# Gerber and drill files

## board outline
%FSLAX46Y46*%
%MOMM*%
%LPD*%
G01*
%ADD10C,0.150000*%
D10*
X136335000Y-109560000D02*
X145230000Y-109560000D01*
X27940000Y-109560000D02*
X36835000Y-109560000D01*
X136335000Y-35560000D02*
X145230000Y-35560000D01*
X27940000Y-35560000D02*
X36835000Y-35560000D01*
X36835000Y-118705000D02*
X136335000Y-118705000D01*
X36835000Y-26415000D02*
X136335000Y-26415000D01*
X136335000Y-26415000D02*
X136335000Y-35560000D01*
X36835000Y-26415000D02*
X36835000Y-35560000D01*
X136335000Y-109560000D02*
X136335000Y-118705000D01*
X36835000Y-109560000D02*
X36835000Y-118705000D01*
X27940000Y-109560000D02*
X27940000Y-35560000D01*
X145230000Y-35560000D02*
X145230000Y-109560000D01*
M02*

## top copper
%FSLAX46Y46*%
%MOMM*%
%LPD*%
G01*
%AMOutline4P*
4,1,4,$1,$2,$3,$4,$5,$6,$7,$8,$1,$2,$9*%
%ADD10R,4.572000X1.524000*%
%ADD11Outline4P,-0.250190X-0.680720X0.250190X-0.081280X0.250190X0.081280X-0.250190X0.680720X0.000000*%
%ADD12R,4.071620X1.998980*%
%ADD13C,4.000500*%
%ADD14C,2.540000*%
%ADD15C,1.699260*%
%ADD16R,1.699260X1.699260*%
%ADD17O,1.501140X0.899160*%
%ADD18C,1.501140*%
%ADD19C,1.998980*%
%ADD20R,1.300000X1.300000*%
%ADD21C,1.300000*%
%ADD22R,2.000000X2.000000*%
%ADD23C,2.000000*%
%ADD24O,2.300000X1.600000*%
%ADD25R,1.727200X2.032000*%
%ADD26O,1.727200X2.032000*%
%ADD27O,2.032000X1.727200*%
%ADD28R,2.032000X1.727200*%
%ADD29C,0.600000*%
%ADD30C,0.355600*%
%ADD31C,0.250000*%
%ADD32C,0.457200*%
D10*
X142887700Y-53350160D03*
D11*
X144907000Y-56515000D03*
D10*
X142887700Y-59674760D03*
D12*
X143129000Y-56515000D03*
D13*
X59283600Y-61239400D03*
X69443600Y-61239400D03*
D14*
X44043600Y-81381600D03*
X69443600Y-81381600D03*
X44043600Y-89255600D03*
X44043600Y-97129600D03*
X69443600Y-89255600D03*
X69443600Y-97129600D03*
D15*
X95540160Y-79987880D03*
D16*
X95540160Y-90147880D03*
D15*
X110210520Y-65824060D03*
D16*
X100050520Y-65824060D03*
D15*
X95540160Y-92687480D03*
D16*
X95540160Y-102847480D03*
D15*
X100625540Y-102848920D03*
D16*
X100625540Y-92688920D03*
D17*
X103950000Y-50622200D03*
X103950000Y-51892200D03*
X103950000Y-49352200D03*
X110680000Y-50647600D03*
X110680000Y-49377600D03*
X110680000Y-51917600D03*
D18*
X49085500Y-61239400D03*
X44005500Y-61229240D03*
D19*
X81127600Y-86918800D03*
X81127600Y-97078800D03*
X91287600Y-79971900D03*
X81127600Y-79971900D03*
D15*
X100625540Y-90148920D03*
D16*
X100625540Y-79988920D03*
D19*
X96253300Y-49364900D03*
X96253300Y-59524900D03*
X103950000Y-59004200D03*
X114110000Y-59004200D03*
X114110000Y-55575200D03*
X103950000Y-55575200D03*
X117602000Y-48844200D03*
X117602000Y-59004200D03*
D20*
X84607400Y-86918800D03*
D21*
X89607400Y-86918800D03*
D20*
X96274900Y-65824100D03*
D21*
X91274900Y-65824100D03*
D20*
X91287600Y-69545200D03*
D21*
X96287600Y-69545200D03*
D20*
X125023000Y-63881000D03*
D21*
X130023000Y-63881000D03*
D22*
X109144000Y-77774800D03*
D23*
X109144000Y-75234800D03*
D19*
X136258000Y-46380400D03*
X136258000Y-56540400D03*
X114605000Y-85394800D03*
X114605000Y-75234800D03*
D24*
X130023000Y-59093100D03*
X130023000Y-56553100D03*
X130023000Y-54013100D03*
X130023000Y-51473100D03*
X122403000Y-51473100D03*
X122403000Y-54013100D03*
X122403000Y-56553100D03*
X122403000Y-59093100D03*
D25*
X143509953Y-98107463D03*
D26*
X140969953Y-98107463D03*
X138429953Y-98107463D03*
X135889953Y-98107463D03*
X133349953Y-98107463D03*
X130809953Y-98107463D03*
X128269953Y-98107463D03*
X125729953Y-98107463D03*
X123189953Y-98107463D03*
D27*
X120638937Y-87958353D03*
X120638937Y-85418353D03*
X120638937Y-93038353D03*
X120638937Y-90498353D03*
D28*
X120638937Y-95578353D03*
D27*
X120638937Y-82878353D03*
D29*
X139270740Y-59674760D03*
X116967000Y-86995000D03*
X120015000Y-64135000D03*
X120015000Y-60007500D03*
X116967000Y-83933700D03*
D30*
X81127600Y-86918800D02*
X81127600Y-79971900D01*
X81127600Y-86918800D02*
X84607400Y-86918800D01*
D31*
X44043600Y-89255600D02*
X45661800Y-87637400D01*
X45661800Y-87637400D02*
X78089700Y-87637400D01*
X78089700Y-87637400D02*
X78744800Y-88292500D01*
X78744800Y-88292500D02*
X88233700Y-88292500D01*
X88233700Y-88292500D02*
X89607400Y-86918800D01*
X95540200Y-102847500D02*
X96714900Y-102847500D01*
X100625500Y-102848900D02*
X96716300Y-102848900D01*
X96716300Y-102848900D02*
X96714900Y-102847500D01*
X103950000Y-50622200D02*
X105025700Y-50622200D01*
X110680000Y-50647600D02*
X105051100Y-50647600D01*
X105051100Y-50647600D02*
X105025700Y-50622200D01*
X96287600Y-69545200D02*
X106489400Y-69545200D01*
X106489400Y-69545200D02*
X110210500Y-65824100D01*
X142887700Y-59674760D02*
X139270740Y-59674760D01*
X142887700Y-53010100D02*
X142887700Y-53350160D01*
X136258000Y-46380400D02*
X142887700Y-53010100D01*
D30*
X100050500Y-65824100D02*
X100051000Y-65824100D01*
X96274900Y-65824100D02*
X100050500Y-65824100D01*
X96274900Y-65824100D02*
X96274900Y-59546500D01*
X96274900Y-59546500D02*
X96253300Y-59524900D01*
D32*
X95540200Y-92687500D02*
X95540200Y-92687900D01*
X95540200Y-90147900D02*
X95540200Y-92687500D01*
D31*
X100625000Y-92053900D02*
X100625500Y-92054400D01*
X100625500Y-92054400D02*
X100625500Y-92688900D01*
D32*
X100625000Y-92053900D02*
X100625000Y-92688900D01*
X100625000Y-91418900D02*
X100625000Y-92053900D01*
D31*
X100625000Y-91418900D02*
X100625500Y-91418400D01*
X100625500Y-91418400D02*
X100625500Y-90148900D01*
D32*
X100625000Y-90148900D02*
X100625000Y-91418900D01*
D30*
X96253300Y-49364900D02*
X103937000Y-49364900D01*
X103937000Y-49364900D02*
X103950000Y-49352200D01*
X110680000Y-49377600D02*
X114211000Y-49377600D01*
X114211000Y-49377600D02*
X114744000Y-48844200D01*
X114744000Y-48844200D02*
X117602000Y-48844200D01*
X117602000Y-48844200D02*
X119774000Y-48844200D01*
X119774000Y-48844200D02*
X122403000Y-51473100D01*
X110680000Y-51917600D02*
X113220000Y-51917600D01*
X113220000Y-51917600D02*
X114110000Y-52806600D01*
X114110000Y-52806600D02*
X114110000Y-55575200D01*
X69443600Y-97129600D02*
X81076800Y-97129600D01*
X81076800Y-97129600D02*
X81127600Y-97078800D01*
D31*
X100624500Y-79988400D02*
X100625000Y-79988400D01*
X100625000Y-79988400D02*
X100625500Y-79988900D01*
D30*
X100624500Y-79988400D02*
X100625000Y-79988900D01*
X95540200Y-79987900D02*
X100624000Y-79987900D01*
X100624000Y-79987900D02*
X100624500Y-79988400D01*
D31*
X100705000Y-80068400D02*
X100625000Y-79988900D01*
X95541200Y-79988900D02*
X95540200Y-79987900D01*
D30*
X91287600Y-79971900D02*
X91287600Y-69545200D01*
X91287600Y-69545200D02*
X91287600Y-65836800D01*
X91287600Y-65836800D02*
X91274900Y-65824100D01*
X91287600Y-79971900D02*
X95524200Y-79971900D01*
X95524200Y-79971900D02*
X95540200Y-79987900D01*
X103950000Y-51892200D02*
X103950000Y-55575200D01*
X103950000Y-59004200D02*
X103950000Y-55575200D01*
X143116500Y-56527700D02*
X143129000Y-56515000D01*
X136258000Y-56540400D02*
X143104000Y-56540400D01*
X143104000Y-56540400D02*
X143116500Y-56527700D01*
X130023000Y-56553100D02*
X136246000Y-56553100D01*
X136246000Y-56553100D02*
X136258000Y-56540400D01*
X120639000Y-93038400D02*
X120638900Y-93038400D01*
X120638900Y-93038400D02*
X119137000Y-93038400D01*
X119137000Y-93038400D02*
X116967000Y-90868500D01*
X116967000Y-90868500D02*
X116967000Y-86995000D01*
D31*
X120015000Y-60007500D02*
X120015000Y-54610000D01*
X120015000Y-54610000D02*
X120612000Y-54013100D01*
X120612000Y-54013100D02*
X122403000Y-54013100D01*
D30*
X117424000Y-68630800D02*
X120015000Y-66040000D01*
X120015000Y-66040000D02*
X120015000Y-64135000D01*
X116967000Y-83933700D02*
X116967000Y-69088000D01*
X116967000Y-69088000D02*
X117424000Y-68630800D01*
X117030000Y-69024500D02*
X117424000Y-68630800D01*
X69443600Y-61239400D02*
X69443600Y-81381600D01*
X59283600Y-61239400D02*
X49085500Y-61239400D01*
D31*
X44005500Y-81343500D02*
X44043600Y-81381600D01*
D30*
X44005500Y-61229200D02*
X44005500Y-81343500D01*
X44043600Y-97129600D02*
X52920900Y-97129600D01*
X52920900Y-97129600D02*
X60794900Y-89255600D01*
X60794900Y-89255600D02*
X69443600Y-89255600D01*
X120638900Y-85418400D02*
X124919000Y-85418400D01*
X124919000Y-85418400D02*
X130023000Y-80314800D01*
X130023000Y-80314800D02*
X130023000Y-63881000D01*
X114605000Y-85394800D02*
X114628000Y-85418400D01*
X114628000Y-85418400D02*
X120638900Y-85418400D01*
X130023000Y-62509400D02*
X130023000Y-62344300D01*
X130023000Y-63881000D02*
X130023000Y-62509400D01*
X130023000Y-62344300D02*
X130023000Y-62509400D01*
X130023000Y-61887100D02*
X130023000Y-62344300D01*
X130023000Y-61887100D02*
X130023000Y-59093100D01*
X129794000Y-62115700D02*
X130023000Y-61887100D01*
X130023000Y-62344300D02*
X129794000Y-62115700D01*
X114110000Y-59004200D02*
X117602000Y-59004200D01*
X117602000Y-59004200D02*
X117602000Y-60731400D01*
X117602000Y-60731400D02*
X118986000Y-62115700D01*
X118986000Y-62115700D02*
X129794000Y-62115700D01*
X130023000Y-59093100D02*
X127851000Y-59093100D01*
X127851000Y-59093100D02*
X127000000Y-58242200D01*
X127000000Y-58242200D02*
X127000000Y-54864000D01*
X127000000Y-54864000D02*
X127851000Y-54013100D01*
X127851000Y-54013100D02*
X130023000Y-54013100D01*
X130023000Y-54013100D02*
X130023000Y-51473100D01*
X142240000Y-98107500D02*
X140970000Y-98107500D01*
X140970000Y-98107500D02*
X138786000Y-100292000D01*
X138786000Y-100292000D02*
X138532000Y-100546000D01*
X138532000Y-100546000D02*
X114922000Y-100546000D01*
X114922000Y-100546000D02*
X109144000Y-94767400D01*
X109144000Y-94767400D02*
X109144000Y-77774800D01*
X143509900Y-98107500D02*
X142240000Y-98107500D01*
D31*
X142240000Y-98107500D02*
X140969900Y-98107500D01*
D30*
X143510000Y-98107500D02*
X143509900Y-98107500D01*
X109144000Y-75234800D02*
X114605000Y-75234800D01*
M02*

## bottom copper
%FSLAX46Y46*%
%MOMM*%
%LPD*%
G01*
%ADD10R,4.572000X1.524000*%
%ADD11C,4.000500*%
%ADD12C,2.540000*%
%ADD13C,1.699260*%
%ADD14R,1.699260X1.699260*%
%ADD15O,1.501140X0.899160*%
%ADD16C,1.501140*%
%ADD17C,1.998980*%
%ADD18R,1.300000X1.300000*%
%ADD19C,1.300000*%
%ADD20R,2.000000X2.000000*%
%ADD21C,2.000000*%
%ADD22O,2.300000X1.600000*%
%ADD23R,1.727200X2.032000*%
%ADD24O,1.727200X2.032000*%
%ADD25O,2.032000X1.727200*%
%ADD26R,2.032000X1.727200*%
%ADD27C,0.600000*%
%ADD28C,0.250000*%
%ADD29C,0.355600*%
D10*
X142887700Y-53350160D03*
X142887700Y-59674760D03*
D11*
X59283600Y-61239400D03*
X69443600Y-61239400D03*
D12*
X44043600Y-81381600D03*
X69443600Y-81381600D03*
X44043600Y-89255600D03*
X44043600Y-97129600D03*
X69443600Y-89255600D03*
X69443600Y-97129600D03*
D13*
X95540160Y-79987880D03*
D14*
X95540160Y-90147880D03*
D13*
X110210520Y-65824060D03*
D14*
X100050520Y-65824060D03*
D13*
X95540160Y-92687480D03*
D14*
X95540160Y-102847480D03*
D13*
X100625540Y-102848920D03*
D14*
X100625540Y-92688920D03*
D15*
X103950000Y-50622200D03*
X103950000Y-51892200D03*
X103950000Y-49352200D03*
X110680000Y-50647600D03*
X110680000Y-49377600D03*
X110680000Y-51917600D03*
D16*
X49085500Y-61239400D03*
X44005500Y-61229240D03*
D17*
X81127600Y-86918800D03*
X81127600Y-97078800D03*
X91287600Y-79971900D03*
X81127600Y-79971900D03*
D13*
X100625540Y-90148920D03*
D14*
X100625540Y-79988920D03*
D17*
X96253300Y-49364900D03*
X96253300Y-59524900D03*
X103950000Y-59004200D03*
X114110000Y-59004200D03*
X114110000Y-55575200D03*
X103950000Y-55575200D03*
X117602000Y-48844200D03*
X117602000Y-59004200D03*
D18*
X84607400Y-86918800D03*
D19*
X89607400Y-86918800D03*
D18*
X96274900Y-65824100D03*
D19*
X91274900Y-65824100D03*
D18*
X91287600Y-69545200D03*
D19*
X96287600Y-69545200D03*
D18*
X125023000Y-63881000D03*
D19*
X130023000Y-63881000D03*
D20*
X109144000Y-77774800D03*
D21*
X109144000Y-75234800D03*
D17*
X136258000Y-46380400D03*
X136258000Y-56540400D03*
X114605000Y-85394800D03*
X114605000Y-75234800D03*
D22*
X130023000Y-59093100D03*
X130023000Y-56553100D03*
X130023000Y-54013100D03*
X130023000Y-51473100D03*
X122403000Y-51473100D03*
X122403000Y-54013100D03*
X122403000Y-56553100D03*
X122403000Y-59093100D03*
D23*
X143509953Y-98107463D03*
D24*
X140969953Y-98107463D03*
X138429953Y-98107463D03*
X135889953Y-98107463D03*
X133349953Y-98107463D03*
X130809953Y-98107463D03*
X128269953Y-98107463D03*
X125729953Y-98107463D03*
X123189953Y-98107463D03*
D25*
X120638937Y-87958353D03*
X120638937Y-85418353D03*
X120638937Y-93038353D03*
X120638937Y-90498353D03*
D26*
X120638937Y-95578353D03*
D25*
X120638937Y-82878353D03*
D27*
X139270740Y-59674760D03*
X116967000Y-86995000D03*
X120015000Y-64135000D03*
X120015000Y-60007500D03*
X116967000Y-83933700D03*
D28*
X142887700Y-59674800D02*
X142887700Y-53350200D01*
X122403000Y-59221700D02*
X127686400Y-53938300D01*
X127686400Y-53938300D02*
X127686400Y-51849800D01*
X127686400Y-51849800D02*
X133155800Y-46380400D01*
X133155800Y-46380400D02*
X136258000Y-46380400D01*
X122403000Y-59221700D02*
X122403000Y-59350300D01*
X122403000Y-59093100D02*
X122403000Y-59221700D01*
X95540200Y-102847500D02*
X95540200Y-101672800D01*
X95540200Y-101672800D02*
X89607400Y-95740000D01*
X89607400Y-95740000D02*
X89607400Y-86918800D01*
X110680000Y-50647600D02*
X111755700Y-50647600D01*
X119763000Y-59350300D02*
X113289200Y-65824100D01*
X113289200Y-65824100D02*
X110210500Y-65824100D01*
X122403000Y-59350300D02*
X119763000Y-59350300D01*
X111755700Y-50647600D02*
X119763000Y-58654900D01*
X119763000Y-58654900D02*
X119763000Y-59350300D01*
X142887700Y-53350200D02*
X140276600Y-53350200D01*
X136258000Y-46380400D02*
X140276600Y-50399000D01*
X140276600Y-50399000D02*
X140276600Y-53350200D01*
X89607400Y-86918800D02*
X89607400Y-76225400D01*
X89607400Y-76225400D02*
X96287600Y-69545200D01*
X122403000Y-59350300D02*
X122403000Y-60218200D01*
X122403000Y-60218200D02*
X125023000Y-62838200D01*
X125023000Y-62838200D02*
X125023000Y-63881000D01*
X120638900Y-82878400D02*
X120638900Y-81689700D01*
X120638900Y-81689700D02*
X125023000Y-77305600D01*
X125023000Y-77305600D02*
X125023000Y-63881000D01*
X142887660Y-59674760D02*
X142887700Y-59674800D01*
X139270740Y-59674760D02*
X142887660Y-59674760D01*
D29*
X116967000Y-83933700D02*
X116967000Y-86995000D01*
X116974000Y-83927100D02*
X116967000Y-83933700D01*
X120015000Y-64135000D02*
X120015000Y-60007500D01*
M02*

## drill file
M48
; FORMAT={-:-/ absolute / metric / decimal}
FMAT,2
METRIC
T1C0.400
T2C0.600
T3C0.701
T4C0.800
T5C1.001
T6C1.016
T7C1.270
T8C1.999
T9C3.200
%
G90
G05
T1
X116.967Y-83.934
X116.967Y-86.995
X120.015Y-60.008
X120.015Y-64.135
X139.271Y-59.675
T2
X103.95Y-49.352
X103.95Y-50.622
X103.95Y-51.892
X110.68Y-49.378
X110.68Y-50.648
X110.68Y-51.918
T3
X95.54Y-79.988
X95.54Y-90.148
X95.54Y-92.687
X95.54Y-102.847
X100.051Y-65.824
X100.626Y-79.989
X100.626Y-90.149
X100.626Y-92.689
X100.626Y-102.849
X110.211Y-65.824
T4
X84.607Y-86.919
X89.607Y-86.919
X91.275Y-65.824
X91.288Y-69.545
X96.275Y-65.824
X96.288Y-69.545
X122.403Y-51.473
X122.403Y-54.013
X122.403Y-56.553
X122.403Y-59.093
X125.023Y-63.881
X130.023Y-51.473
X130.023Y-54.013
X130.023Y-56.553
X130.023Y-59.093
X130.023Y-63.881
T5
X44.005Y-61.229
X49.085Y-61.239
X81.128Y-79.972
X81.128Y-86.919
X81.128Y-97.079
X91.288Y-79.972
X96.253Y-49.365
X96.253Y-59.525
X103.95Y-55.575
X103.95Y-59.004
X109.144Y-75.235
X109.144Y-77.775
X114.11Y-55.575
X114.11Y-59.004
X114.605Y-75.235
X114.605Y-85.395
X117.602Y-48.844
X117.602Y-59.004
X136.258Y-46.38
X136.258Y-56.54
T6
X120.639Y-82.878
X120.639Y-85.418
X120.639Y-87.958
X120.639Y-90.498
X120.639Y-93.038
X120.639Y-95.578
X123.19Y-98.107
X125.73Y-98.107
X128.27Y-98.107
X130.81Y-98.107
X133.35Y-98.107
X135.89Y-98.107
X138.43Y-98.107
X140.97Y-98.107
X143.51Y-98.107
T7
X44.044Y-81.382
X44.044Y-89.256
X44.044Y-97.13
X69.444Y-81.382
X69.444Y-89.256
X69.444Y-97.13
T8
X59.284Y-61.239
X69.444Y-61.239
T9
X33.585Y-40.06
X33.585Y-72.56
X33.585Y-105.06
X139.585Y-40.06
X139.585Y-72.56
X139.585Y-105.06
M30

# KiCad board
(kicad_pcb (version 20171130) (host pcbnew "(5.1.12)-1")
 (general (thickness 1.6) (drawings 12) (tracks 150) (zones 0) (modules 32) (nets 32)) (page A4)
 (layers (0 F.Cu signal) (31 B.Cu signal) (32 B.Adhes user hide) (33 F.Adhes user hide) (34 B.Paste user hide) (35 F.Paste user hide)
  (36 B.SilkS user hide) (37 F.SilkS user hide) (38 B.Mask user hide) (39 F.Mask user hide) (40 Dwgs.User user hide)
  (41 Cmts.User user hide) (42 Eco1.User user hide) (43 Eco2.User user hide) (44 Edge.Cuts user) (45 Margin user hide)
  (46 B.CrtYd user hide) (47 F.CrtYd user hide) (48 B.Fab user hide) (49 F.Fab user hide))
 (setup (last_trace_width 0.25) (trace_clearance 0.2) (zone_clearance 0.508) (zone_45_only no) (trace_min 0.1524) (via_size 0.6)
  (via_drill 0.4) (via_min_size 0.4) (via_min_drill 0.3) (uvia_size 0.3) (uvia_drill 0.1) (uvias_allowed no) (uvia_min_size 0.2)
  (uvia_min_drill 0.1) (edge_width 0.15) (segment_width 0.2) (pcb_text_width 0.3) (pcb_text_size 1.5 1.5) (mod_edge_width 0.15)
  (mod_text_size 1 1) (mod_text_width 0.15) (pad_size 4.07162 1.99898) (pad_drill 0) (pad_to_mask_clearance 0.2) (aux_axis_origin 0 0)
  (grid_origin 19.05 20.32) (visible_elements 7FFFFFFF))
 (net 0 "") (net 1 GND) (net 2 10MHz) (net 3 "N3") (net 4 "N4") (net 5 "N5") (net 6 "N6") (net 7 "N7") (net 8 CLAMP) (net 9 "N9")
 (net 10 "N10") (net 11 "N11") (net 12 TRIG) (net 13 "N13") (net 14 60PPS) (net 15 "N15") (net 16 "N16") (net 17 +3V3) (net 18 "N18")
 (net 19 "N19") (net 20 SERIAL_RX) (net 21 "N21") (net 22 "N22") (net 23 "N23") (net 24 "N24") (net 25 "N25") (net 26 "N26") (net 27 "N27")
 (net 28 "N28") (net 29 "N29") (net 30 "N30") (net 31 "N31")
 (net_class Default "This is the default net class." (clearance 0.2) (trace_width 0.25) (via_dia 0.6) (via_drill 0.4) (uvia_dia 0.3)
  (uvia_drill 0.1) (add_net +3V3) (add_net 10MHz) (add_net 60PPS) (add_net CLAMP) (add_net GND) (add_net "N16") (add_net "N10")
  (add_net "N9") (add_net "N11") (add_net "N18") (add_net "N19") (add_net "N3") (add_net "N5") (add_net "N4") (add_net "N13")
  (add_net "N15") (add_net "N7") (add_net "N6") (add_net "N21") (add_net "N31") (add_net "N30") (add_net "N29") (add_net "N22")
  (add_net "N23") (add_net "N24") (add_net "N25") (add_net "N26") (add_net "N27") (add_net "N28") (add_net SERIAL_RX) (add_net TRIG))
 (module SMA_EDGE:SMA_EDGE (layer F.Cu) (at 151.765 55.245)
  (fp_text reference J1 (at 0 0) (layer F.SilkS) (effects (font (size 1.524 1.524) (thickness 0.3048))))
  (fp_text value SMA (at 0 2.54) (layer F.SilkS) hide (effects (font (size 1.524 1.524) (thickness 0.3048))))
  (pad 0 connect rect (at -8.8773 -1.89484) (size 4.572 1.524) (layers *.Cu F.Mask) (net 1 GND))
  (pad 1 connect trapezoid (at -6.858 1.27) (size 0.50038 0.762) (rect_delta 0.59944 0) (layers F.Cu F.Mask) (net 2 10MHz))
  (pad 2 connect rect (at -8.8773 4.42976) (size 4.572 1.524) (layers *.Cu F.Mask) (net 1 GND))
  (pad 1 connect rect (at -8.636 1.27) (size 4.07162 1.99898) (layers F.Cu F.Mask) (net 2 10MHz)))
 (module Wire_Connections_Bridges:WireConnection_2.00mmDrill (layer F.Cu) (at 59.2836 61.2394)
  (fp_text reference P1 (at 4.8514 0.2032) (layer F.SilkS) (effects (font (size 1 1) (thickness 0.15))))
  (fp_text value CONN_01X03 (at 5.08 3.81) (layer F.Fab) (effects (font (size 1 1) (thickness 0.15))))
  (pad 1 thru_hole circle (at 0 0) (size 4.0005 4.0005) (drill 1.99898) (layers *.Cu *.Mask F.SilkS) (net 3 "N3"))
  (pad 2 thru_hole circle (at 10.16 0) (size 4.0005 4.0005) (drill 1.99898) (layers *.Cu *.Mask F.SilkS) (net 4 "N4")))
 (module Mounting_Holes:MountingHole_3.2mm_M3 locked (layer F.Cu) (at 139.585 105.06)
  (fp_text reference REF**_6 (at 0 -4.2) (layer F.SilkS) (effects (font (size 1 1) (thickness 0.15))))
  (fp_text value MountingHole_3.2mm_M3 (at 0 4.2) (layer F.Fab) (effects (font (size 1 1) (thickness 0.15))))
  (pad 1 np_thru_hole circle (at 0 0) (size 3.2 3.2) (drill 3.2) (layers *.Cu *.Mask F.SilkS)))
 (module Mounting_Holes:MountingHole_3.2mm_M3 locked (layer F.Cu) (at 139.585 72.56)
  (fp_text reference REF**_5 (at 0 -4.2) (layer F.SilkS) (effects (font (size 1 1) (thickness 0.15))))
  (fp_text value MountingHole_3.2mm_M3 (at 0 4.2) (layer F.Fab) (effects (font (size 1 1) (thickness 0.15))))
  (pad 1 np_thru_hole circle (at 0 0) (size 3.2 3.2) (drill 3.2) (layers *.Cu *.Mask F.SilkS)))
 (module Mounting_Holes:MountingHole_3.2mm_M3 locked (layer F.Cu) (at 33.585 105.06)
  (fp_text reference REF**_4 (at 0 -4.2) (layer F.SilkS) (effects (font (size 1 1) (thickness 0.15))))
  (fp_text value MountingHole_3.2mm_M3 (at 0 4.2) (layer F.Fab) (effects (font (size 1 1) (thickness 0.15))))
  (pad 1 np_thru_hole circle (at 0 0) (size 3.2 3.2) (drill 3.2) (layers *.Cu *.Mask F.SilkS)))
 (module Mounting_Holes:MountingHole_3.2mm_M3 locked (layer F.Cu) (at 33.585 72.56)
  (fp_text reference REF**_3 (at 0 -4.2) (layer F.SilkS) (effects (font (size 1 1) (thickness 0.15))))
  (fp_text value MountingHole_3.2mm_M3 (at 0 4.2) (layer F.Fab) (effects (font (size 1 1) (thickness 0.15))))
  (pad 1 np_thru_hole circle (at 0 0) (size 3.2 3.2) (drill 3.2) (layers *.Cu *.Mask F.SilkS)))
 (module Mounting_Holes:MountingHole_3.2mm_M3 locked (layer F.Cu) (at 139.585 40.06)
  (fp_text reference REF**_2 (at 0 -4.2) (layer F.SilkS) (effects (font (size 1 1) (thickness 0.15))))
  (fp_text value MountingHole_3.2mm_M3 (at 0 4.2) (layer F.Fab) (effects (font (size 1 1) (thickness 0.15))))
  (pad 1 np_thru_hole circle (at 0 0) (size 3.2 3.2) (drill 3.2) (layers *.Cu *.Mask F.SilkS)))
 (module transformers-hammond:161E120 (layer F.Cu) (at 41.5036 71.2216)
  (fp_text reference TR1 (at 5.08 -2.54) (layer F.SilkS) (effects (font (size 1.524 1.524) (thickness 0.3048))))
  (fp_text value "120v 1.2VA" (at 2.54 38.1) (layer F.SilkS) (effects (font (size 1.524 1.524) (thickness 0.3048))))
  (pad 1 thru_hole circle (at 2.54 10.16) (size 2.54 2.54) (drill 1.27) (layers *.Cu *.Mask F.SilkS) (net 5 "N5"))
  (pad 2 thru_hole circle (at 27.94 10.16) (size 2.54 2.54) (drill 1.27) (layers *.Cu *.SilkS *.Mask) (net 4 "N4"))
  (pad 3 thru_hole circle (at 2.54 18.034) (size 2.54 2.54) (drill 1.27) (layers *.Cu *.SilkS *.Mask) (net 1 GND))
  (pad 4 thru_hole circle (at 2.54 25.908) (size 2.54 2.54) (drill 1.27) (layers *.Cu *.SilkS *.Mask) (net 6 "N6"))
  (pad 5 thru_hole circle (at 27.94 18.034) (size 2.54 2.54) (drill 1.27) (layers *.Cu *.SilkS *.Mask) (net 6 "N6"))
  (pad 6 thru_hole circle (at 27.94 25.908) (size 2.54 2.54) (drill 1.27) (layers *.Cu *.SilkS *.Mask) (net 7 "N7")))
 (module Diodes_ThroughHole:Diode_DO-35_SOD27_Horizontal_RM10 (layer F.Cu) (at 95.5427 90.1484 90)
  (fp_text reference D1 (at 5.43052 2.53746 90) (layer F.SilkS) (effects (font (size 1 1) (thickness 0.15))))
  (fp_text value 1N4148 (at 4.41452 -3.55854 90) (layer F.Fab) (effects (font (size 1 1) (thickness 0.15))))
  (pad 2 thru_hole circle (at 10.16052 -0.00254 270) (size 1.69926 1.69926) (drill 0.70104) (layers *.Cu *.Mask F.SilkS) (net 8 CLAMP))
  (pad 1 thru_hole rect (at 0.00052 -0.00254 270) (size 1.69926 1.69926) (drill 0.70104) (layers *.Cu *.Mask F.SilkS) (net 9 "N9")))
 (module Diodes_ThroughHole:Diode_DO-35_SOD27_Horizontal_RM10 (layer F.Cu) (at 100.05 65.8266)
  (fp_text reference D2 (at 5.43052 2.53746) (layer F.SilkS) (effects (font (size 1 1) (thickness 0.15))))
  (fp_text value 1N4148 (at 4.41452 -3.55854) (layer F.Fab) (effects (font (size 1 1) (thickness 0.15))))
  (pad 2 thru_hole circle (at 10.16052 -0.00254 180) (size 1.69926 1.69926) (drill 0.70104) (layers *.Cu *.Mask F.SilkS) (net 1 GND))
  (pad 1 thru_hole rect (at 0.00052 -0.00254 180) (size 1.69926 1.69926) (drill 0.70104) (layers *.Cu *.Mask F.SilkS) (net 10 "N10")))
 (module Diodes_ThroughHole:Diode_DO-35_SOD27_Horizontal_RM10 (layer F.Cu) (at 95.5427 102.848 90)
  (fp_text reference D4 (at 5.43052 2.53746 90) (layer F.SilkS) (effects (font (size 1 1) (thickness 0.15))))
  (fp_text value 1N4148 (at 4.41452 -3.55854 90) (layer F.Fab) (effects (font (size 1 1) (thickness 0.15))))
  (pad 2 thru_hole circle (at 10.16052 -0.00254 270) (size 1.69926 1.69926) (drill 0.70104) (layers *.Cu *.Mask F.SilkS) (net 9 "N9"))
  (pad 1 thru_hole rect (at 0.00052 -0.00254 270) (size 1.69926 1.69926) (drill 0.70104) (layers *.Cu *.Mask F.SilkS) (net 1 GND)))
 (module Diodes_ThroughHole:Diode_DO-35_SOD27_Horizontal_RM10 (layer F.Cu) (at 100.623 92.6884 270)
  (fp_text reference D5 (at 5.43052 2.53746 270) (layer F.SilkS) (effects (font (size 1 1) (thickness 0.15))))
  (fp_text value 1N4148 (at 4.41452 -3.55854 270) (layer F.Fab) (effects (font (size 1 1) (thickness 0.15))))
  (pad 2 thru_hole circle (at 10.16052 -0.00254 90) (size 1.69926 1.69926) (drill 0.70104) (layers *.Cu *.Mask F.SilkS) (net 1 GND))
  (pad 1 thru_hole rect (at 0.00052 -0.00254 90) (size 1.69926 1.69926) (drill 0.70104) (layers *.Cu *.Mask F.SilkS) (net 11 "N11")))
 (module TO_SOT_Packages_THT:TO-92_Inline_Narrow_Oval (layer F.Cu) (at 103.95 49.3522 270)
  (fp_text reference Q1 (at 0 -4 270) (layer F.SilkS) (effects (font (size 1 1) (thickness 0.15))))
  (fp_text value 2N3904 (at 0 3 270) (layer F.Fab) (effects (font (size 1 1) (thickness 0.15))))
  (pad 2 thru_hole oval (at 1.27 0 90) (size 0.89916 1.50114) (drill 0.6) (layers *.Cu *.Mask F.SilkS) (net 1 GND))
  (pad 3 thru_hole oval (at 2.54 0 90) (size 0.89916 1.50114) (drill 0.6) (layers *.Cu *.Mask F.SilkS) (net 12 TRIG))
  (pad 1 thru_hole oval (at 0 0 90) (size 0.89916 1.50114) (drill 0.6) (layers *.Cu *.Mask F.SilkS) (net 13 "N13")))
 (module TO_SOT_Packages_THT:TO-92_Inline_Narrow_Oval (layer F.Cu) (at 110.68 51.9176 90)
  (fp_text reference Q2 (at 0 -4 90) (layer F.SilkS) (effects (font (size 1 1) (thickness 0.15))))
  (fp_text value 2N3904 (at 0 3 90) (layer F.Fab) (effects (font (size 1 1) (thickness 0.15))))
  (pad 2 thru_hole oval (at 1.27 0 270) (size 0.89916 1.50114) (drill 0.6) (layers *.Cu *.Mask F.SilkS) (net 1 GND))
  (pad 3 thru_hole oval (at 2.54 0 270) (size 0.89916 1.50114) (drill 0.6) (layers *.Cu *.Mask F.SilkS) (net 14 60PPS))
  (pad 1 thru_hole oval (at 0 0 270) (size 0.89916 1.50114) (drill 0.6) (layers *.Cu *.Mask F.SilkS) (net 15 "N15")))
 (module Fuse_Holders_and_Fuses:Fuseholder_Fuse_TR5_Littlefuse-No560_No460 (layer F.Cu) (at 46.5455 61.2394 180)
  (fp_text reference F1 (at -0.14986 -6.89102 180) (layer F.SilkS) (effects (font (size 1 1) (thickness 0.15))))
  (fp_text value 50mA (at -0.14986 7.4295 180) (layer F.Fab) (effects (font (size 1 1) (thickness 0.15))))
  (pad 1 thru_hole circle (at -2.54 0 180) (size 1.50114 1.50114) (drill 1.00076) (layers *.Cu *.Mask F.SilkS) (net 3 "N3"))
  (pad 2 thru_hole circle (at 2.54 0.01016 180) (size 1.50114 1.50114) (drill 1.00076) (layers *.Cu *.Mask F.SilkS) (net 5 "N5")))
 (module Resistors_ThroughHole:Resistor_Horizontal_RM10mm (layer F.Cu) (at 81.1276 86.9188 270)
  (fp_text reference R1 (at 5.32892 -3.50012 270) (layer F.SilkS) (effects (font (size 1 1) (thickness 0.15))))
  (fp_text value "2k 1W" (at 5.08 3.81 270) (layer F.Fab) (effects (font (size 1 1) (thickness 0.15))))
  (pad 1 thru_hole circle (at 0 0 270) (size 1.99898 1.99898) (drill 1.00076) (layers *.Cu *.SilkS *.Mask) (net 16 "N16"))
  (pad 2 thru_hole circle (at 10.16 0 270) (size 1.99898 1.99898) (drill 1.00076) (layers *.Cu *.SilkS *.Mask) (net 7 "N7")))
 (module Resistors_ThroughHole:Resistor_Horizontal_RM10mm (layer F.Cu) (at 91.2876 79.9719 180)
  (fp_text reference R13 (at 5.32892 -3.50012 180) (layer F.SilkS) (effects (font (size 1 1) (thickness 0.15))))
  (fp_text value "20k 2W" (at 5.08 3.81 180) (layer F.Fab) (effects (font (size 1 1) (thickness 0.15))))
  (pad 1 thru_hole circle (at 0 0 180) (size 1.99898 1.99898) (drill 1.00076) (layers *.Cu *.SilkS *.Mask) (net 8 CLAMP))
  (pad 2 thru_hole circle (at 10.16 0 180) (size 1.99898 1.99898) (drill 1.00076) (layers *.Cu *.SilkS *.Mask) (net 16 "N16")))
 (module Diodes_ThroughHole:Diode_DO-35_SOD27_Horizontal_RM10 (layer F.Cu) (at 100.623 79.9884 270)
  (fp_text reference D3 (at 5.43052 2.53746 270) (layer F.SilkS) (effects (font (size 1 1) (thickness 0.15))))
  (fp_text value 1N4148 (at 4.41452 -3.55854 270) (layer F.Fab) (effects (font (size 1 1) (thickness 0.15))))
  (pad 2 thru_hole circle (at 10.16052 -0.00254 90) (size 1.69926 1.69926) (drill 0.70104) (layers *.Cu *.Mask F.SilkS) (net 11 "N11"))
  (pad 1 thru_hole rect (at 0.00052 -0.00254 90) (size 1.69926 1.69926) (drill 0.70104) (layers *.Cu *.Mask F.SilkS) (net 8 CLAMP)))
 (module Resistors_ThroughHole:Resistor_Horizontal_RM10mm (layer F.Cu) (at 96.2533 49.3649 270)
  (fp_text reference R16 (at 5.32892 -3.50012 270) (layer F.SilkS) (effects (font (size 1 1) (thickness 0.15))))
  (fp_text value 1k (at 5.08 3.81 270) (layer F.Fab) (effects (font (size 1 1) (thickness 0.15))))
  (pad 1 thru_hole circle (at 0 0 270) (size 1.99898 1.99898) (drill 1.00076) (layers *.Cu *.SilkS *.Mask) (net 13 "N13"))
  (pad 2 thru_hole circle (at 10.16 0 270) (size 1.99898 1.99898) (drill 1.00076) (layers *.Cu *.SilkS *.Mask) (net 10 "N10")))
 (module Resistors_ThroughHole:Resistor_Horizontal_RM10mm (layer F.Cu) (at 103.95 59.0042)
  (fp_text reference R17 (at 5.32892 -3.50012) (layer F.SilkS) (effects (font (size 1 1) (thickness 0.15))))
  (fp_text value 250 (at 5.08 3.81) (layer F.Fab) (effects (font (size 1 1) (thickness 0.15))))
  (pad 1 thru_hole circle (at 0 0) (size 1.99898 1.99898) (drill 1.00076) (layers *.Cu *.SilkS *.Mask) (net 12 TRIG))
  (pad 2 thru_hole circle (at 10.16 0) (size 1.99898 1.99898) (drill 1.00076) (layers *.Cu *.SilkS *.Mask) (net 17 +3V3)))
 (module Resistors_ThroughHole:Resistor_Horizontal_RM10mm (layer F.Cu) (at 114.11 55.5752 180)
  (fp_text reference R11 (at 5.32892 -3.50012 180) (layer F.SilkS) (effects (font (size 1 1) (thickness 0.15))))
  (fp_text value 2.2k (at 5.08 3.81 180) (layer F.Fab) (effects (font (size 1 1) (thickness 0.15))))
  (pad 1 thru_hole circle (at 0 0 180) (size 1.99898 1.99898) (drill 1.00076) (layers *.Cu *.SilkS *.Mask) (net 15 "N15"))
  (pad 2 thru_hole circle (at 10.16 0 180) (size 1.99898 1.99898) (drill 1.00076) (layers *.Cu *.SilkS *.Mask) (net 12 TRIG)))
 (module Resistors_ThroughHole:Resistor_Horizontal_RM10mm (layer F.Cu) (at 117.602 48.8442 270)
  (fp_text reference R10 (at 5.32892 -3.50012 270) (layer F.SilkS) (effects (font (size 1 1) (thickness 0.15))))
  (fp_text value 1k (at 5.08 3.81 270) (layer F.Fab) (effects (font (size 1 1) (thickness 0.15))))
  (pad 1 thru_hole circle (at 0 0 270) (size 1.99898 1.99898) (drill 1.00076) (layers *.Cu *.SilkS *.Mask) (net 14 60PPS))
  (pad 2 thru_hole circle (at 10.16 0 270) (size 1.99898 1.99898) (drill 1.00076) (layers *.Cu *.SilkS *.Mask) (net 17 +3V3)))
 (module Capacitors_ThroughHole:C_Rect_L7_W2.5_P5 (layer F.Cu) (at 84.6074 86.9188)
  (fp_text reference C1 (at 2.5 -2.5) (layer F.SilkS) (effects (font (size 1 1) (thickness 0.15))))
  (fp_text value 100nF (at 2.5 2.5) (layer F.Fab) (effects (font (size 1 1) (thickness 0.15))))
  (pad 1 thru_hole rect (at 0 0) (size 1.3 1.3) (drill 0.8) (layers *.Cu *.Mask F.SilkS) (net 16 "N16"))
  (pad 2 thru_hole circle (at 5 0) (size 1.3 1.3) (drill 0.8) (layers *.Cu *.Mask F.SilkS) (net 1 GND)))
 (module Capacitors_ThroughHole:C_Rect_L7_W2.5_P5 (layer F.Cu) (at 96.2749 65.8241 180)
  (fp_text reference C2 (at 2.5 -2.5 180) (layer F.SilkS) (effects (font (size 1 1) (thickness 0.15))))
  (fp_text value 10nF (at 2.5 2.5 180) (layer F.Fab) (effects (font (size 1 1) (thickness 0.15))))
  (pad 1 thru_hole rect (at 0 0 180) (size 1.3 1.3) (drill 0.8) (layers *.Cu *.Mask F.SilkS) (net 10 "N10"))
  (pad 2 thru_hole circle (at 5 0 180) (size 1.3 1.3) (drill 0.8) (layers *.Cu *.Mask F.SilkS) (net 8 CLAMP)))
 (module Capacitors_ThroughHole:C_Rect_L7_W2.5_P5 (layer F.Cu) (at 91.2876 69.5452)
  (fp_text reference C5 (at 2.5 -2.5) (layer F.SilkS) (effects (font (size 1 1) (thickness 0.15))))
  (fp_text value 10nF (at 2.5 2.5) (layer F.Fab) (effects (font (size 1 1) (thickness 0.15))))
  (pad 1 thru_hole rect (at 0 0) (size 1.3 1.3) (drill 0.8) (layers *.Cu *.Mask F.SilkS) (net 8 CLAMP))
  (pad 2 thru_hole circle (at 5 0) (size 1.3 1.3) (drill 0.8) (layers *.Cu *.Mask F.SilkS) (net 1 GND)))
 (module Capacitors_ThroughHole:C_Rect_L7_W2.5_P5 (layer F.Cu) (at 125.023 63.881)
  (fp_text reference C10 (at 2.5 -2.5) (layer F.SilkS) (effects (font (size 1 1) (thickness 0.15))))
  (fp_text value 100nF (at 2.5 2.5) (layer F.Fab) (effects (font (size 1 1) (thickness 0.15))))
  (pad 1 thru_hole rect (at 0 0) (size 1.3 1.3) (drill 0.8) (layers *.Cu *.Mask F.SilkS) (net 1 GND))
  (pad 2 thru_hole circle (at 5 0) (size 1.3 1.3) (drill 0.8) (layers *.Cu *.Mask F.SilkS) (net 17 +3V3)))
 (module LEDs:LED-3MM (layer F.Cu) (at 109.144 77.7748 90)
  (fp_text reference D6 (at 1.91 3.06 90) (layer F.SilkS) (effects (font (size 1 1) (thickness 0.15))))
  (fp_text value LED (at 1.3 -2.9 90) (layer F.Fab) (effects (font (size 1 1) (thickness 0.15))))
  (pad 1 thru_hole rect (at 0 0 180) (size 2 2) (drill 1.00076) (layers *.Cu *.Mask F.SilkS) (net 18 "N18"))
  (pad 2 thru_hole circle (at 2.54 0 90) (size 2 2) (drill 1.00076) (layers *.Cu *.Mask F.SilkS) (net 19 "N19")))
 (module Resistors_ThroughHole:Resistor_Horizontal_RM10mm (layer F.Cu) (at 136.258 46.3804 270)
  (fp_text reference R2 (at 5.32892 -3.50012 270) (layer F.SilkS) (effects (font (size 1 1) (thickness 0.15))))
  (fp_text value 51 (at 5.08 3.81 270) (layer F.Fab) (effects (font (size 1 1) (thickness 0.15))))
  (pad 1 thru_hole circle (at 0 0 270) (size 1.99898 1.99898) (drill 1.00076) (layers *.Cu *.SilkS *.Mask) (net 1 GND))
  (pad 2 thru_hole circle (at 10.16 0 270) (size 1.99898 1.99898) (drill 1.00076) (layers *.Cu *.SilkS *.Mask) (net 2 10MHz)))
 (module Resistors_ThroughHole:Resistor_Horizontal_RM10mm (layer F.Cu) (at 114.605 85.3948 90)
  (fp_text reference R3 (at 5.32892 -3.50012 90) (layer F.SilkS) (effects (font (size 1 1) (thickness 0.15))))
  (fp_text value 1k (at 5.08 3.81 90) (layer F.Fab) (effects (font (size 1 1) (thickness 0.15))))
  (pad 1 thru_hole circle (at 0 0 90) (size 1.99898 1.99898) (drill 1.00076) (layers *.Cu *.SilkS *.Mask) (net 17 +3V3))
  (pad 2 thru_hole circle (at 10.16 0 90) (size 1.99898 1.99898) (drill 1.00076) (layers *.Cu *.SilkS *.Mask) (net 19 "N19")))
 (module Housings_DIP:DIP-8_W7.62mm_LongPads (layer F.Cu) (at 130.023 59.0931 180)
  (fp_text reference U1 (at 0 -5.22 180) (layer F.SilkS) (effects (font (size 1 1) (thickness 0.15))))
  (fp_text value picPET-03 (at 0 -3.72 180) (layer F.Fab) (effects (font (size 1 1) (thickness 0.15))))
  (pad 1 thru_hole oval (at 0 0 180) (size 2.3 1.6) (drill 0.8) (layers *.Cu *.Mask F.SilkS) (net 17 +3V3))
  (pad 2 thru_hole oval (at 0 2.54 180) (size 2.3 1.6) (drill 0.8) (layers *.Cu *.Mask F.SilkS) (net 2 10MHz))
  (pad 3 thru_hole oval (at 0 5.08 180) (size 2.3 1.6) (drill 0.8) (layers *.Cu *.Mask F.SilkS) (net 17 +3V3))
  (pad 4 thru_hole oval (at 0 7.62 180) (size 2.3 1.6) (drill 0.8) (layers *.Cu *.Mask F.SilkS) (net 17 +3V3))
  (pad 5 thru_hole oval (at 7.62 7.62 180) (size 2.3 1.6) (drill 0.8) (layers *.Cu *.Mask F.SilkS) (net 14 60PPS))
  (pad 6 thru_hole oval (at 7.62 5.08 180) (size 2.3 1.6) (drill 0.8) (layers *.Cu *.Mask F.SilkS) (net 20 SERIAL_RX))
  (pad 7 thru_hole oval (at 7.62 2.54 180) (size 2.3 1.6) (drill 0.8) (layers *.Cu *.Mask F.SilkS) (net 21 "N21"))
  (pad 8 thru_hole oval (at 7.62 0 180) (size 2.3 1.6) (drill 0.8) (layers *.Cu *.Mask F.SilkS) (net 1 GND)))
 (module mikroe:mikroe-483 (layer F.Cu) (at 145.277 99.8854 180)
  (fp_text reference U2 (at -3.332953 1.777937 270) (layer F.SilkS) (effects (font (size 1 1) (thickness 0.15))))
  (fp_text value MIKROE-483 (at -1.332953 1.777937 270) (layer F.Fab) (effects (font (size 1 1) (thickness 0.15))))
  (pad 3-1 thru_hole rect (at 1.767047 1.777937 270) (size 2.032 1.7272) (drill 1.016) (layers *.Cu *.Mask F.SilkS) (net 18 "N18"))
  (pad 3-2 thru_hole oval (at 4.307047 1.777937 270) (size 2.032 1.7272) (drill 1.016) (layers *.Cu *.Mask F.SilkS) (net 18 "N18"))
  (pad 3-3 thru_hole oval (at 6.847047 1.777937 270) (size 2.032 1.7272) (drill 1.016) (layers *.Cu *.Mask F.SilkS) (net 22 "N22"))
  (pad 3-4 thru_hole oval (at 9.387047 1.777937 270) (size 2.032 1.7272) (drill 1.016) (layers *.Cu *.Mask F.SilkS) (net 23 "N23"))
  (pad 3-5 thru_hole oval (at 11.927047 1.777937 90) (size 2.032 1.7272) (drill 1.016) (layers *.Cu *.Mask F.SilkS) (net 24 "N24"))
  (pad 3-6 thru_hole oval (at 14.467047 1.777937 270) (size 2.032 1.7272) (drill 1.016) (layers *.Cu *.Mask F.SilkS) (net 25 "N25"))
  (pad 3-7 thru_hole oval (at 17.007047 1.777937 270) (size 2.032 1.7272) (drill 1.016) (layers *.Cu *.Mask F.SilkS) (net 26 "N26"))
  (pad 3-8 thru_hole oval (at 19.547047 1.777937 270) (size 2.032 1.7272) (drill 1.016) (layers *.Cu *.Mask F.SilkS) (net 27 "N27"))
  (pad 3-9 thru_hole oval (at 22.087047 1.777937 270) (size 2.032 1.7272) (drill 1.016) (layers *.Cu *.Mask F.SilkS) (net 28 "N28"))
  (pad 2-4 thru_hole oval (at 24.638063 11.927047 180) (size 2.032 1.7272) (drill 1.016) (layers *.Cu *.Mask F.SilkS) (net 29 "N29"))
  (pad 2-5 thru_hole oval (at 24.638063 14.467047) (size 2.032 1.7272) (drill 1.016) (layers *.Cu *.Mask F.SilkS) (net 17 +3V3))
  (pad 2-2 thru_hole oval (at 24.638063 6.847047 180) (size 2.032 1.7272) (drill 1.016) (layers *.Cu *.Mask F.SilkS) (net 20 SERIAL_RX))
  (pad 2-3 thru_hole oval (at 24.638063 9.387047 180) (size 2.032 1.7272) (drill 1.016) (layers *.Cu *.Mask F.SilkS) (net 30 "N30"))
  (pad 2-1 thru_hole rect (at 24.638063 4.307047 180) (size 2.032 1.7272) (drill 1.016) (layers *.Cu *.Mask F.SilkS) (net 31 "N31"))
  (pad 2-6 thru_hole oval (at 24.638063 17.007047 180) (size 2.032 1.7272) (drill 1.016) (layers *.Cu *.Mask F.SilkS) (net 1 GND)))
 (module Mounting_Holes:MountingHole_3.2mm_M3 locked (layer F.Cu) (at 33.585 40.06)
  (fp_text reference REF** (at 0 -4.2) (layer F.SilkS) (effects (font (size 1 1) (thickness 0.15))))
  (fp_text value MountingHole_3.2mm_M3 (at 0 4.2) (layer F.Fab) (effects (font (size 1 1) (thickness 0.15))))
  (pad 1 np_thru_hole circle (at 0 0) (size 3.2 3.2) (drill 3.2) (layers *.Cu *.Mask F.SilkS)))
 (gr_line (start 136.335 109.56) (end 145.23 109.56) (layer Edge.Cuts) (width 0.15))
 (gr_line (start 27.94 109.56) (end 36.835 109.56) (layer Edge.Cuts) (width 0.15))
 (gr_line (start 136.335 35.56) (end 145.23 35.56) (layer Edge.Cuts) (width 0.15))
 (gr_line (start 27.94 35.56) (end 36.835 35.56) (layer Edge.Cuts) (width 0.15))
 (gr_line (start 36.835 118.705) (end 136.335 118.705) (layer Edge.Cuts) (width 0.15))
 (gr_line (start 36.835 26.415) (end 136.335 26.415) (layer Edge.Cuts) (width 0.15))
 (gr_line (start 136.335 26.415) (end 136.335 35.56) (layer Edge.Cuts) (width 0.15))
 (gr_line (start 36.835 26.415) (end 36.835 35.56) (layer Edge.Cuts) (width 0.15))
 (gr_line (start 136.335 109.56) (end 136.335 118.705) (layer Edge.Cuts) (width 0.15))
 (gr_line (start 36.835 109.56) (end 36.835 118.705) (layer Edge.Cuts) (width 0.15))
 (gr_line (start 27.94 109.56) (end 27.94 35.56) (layer Edge.Cuts) (width 0.15))
 (gr_line (start 145.23 35.56) (end 145.23 109.56) (layer Edge.Cuts) (width 0.15))
 (via (at 139.27074 59.67476) (size 0.6) (drill 0.4) (layers F.Cu B.Cu) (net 1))
 (segment (start 81.1276 86.9188) (end 81.1276 79.9719) (width 0.3556) (layer F.Cu) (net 16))
 (segment (start 81.1276 86.9188) (end 84.6074 86.9188) (width 0.3556) (layer F.Cu) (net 16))
 (segment (start 142.8877 59.6748) (end 142.8877 53.3502) (width 0.25) (layer B.Cu) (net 1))
 (segment (start 44.0436 89.2556) (end 45.6618 87.6374) (width 0.25) (layer F.Cu) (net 1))
 (segment (start 45.6618 87.6374) (end 78.0897 87.6374) (width 0.25) (layer F.Cu) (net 1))
 (segment (start 78.0897 87.6374) (end 78.7448 88.2925) (width 0.25) (layer F.Cu) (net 1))
 (segment (start 78.7448 88.2925) (end 88.2337 88.2925) (width 0.25) (layer F.Cu) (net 1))
 (segment (start 88.2337 88.2925) (end 89.6074 86.9188) (width 0.25) (layer F.Cu) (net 1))
 (segment (start 122.403 59.2217) (end 127.6864 53.9383) (width 0.25) (layer B.Cu) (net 1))
 (segment (start 127.6864 53.9383) (end 127.6864 51.8498) (width 0.25) (layer B.Cu) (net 1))
 (segment (start 127.6864 51.8498) (end 133.1558 46.3804) (width 0.25) (layer B.Cu) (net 1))
 (segment (start 133.1558 46.3804) (end 136.258 46.3804) (width 0.25) (layer B.Cu) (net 1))
 (segment (start 122.403 59.2217) (end 122.403 59.3503) (width 0.25) (layer B.Cu) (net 1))
 (segment (start 122.403 59.0931) (end 122.403 59.2217) (width 0.25) (layer B.Cu) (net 1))
 (segment (start 95.5402 102.8475) (end 95.5402 101.6728) (width 0.25) (layer B.Cu) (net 1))
 (segment (start 95.5402 101.6728) (end 89.6074 95.74) (width 0.25) (layer B.Cu) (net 1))
 (segment (start 89.6074 95.74) (end 89.6074 86.9188) (width 0.25) (layer B.Cu) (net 1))
 (segment (start 95.5402 102.8475) (end 96.7149 102.8475) (width 0.25) (layer F.Cu) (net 1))
 (segment (start 100.6255 102.8489) (end 96.7163 102.8489) (width 0.25) (layer F.Cu) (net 1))
 (segment (start 96.7163 102.8489) (end 96.7149 102.8475) (width 0.25) (layer F.Cu) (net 1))
 (segment (start 110.68 50.6476) (end 111.7557 50.6476) (width 0.25) (layer B.Cu) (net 1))
 (segment (start 119.763 59.3503) (end 113.2892 65.8241) (width 0.25) (layer B.Cu) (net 1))
 (segment (start 113.2892 65.8241) (end 110.2105 65.8241) (width 0.25) (layer B.Cu) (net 1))
 (segment (start 122.403 59.3503) (end 119.763 59.3503) (width 0.25) (layer B.Cu) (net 1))
 (segment (start 111.7557 50.6476) (end 119.763 58.6549) (width 0.25) (layer B.Cu) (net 1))
 (segment (start 119.763 58.6549) (end 119.763 59.3503) (width 0.25) (layer B.Cu) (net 1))
 (segment (start 103.95 50.6222) (end 105.0257 50.6222) (width 0.25) (layer F.Cu) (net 1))
 (segment (start 110.68 50.6476) (end 105.0511 50.6476) (width 0.25) (layer F.Cu) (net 1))
 (segment (start 105.0511 50.6476) (end 105.0257 50.6222) (width 0.25) (layer F.Cu) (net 1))
 (segment (start 142.8877 53.3502) (end 140.2766 53.3502) (width 0.25) (layer B.Cu) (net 1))
 (segment (start 136.258 46.3804) (end 140.2766 50.399) (width 0.25) (layer B.Cu) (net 1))
 (segment (start 140.2766 50.399) (end 140.2766 53.3502) (width 0.25) (layer B.Cu) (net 1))
 (segment (start 89.6074 86.9188) (end 89.6074 76.2254) (width 0.25) (layer B.Cu) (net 1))
 (segment (start 89.6074 76.2254) (end 96.2876 69.5452) (width 0.25) (layer B.Cu) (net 1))
 (segment (start 96.2876 69.5452) (end 106.4894 69.5452) (width 0.25) (layer F.Cu) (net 1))
 (segment (start 106.4894 69.5452) (end 110.2105 65.8241) (width 0.25) (layer F.Cu) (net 1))
 (segment (start 122.403 59.3503) (end 122.403 60.2182) (width 0.25) (layer B.Cu) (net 1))
 (segment (start 122.403 60.2182) (end 125.023 62.8382) (width 0.25) (layer B.Cu) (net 1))
 (segment (start 125.023 62.8382) (end 125.023 63.881) (width 0.25) (layer B.Cu) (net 1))
 (segment (start 120.6389 82.8784) (end 120.6389 81.6897) (width 0.25) (layer B.Cu) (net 1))
 (segment (start 120.6389 81.6897) (end 125.023 77.3056) (width 0.25) (layer B.Cu) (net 1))
 (segment (start 125.023 77.3056) (end 125.023 63.881) (width 0.25) (layer B.Cu) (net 1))
 (segment (start 142.8877 59.67476) (end 139.27074 59.67476) (width 0.25) (layer F.Cu) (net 1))
 (segment (start 142.88766 59.67476) (end 142.8877 59.6748) (width 0.25) (layer B.Cu) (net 1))
 (segment (start 139.27074 59.67476) (end 142.88766 59.67476) (width 0.25) (layer B.Cu) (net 1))
 (segment (start 142.8877 53.0101) (end 142.8877 53.35016) (width 0.25) (layer F.Cu) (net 1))
 (segment (start 136.258 46.3804) (end 142.8877 53.0101) (width 0.25) (layer F.Cu) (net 1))
 (segment (start 100.0505 65.8241) (end 100.051 65.8241) (width 0.3556) (layer F.Cu) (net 10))
 (segment (start 96.2749 65.8241) (end 100.0505 65.8241) (width 0.3556) (layer F.Cu) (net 10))
 (segment (start 96.2749 65.8241) (end 96.2749 59.5465) (width 0.3556) (layer F.Cu) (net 10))
 (segment (start 96.2749 59.5465) (end 96.2533 59.5249) (width 0.3556) (layer F.Cu) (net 10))
 (segment (start 95.5402 92.6875) (end 95.5402 92.6879) (width 0.4572) (layer F.Cu) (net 9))
 (segment (start 95.5402 90.1479) (end 95.5402 92.6875) (width 0.4572) (layer F.Cu) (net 9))
 (segment (start 100.625 92.0539) (end 100.6255 92.0544) (width 0.25) (layer F.Cu) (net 11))
 (segment (start 100.6255 92.0544) (end 100.6255 92.6889) (width 0.25) (layer F.Cu) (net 11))
 (segment (start 100.625 92.0539) (end 100.625 92.6889) (width 0.4572) (layer F.Cu) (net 11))
 (segment (start 100.625 91.4189) (end 100.625 92.0539) (width 0.4572) (layer F.Cu) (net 11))
 (segment (start 100.625 91.4189) (end 100.6255 91.4184) (width 0.25) (layer F.Cu) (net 11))
 (segment (start 100.6255 91.4184) (end 100.6255 90.1489) (width 0.25) (layer F.Cu) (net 11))
 (segment (start 100.625 90.1489) (end 100.625 91.4189) (width 0.4572) (layer F.Cu) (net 11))
 (segment (start 96.2533 49.3649) (end 103.937 49.3649) (width 0.3556) (layer F.Cu) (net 13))
 (segment (start 103.937 49.3649) (end 103.95 49.3522) (width 0.3556) (layer F.Cu) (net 13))
 (segment (start 110.68 49.3776) (end 114.211 49.3776) (width 0.3556) (layer F.Cu) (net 14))
 (segment (start 114.211 49.3776) (end 114.744 48.8442) (width 0.3556) (layer F.Cu) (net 14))
 (segment (start 114.744 48.8442) (end 117.602 48.8442) (width 0.3556) (layer F.Cu) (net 14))
 (segment (start 117.602 48.8442) (end 119.774 48.8442) (width 0.3556) (layer F.Cu) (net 14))
 (segment (start 119.774 48.8442) (end 122.403 51.4731) (width 0.3556) (layer F.Cu) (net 14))
 (segment (start 110.68 51.9176) (end 113.22 51.9176) (width 0.3556) (layer F.Cu) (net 15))
 (segment (start 113.22 51.9176) (end 114.11 52.8066) (width 0.3556) (layer F.Cu) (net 15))
 (segment (start 114.11 52.8066) (end 114.11 55.5752) (width 0.3556) (layer F.Cu) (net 15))
 (segment (start 69.4436 97.1296) (end 81.0768 97.1296) (width 0.3556) (layer F.Cu) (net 7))
 (segment (start 81.0768 97.1296) (end 81.1276 97.0788) (width 0.3556) (layer F.Cu) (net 7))
 (segment (start 100.6245 79.9884) (end 100.625 79.9884) (width 0.25) (layer F.Cu) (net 8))
 (segment (start 100.625 79.9884) (end 100.6255 79.9889) (width 0.25) (layer F.Cu) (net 8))
 (segment (start 100.6245 79.9884) (end 100.625 79.9889) (width 0.3556) (layer F.Cu) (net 8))
 (segment (start 95.5402 79.9879) (end 100.624 79.9879) (width 0.3556) (layer F.Cu) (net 8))
 (segment (start 100.624 79.9879) (end 100.6245 79.9884) (width 0.3556) (layer F.Cu) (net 8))
 (segment (start 100.705 80.0684) (end 100.625 79.9889) (width 0.25) (layer F.Cu) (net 8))
 (segment (start 95.5412 79.9889) (end 95.5402 79.9879) (width 0.25) (layer F.Cu) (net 8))
 (segment (start 91.2876 79.9719) (end 91.2876 69.5452) (width 0.3556) (layer F.Cu) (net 8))
 (segment (start 91.2876 69.5452) (end 91.2876 65.8368) (width 0.3556) (layer F.Cu) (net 8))
 (segment (start 91.2876 65.8368) (end 91.2749 65.8241) (width 0.3556) (layer F.Cu) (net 8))
 (segment (start 91.2876 79.9719) (end 95.5242 79.9719) (width 0.3556) (layer F.Cu) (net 8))
 (segment (start 95.5242 79.9719) (end 95.5402 79.9879) (width 0.3556) (layer F.Cu) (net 8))
 (segment (start 103.95 51.8922) (end 103.95 55.5752) (width 0.3556) (layer F.Cu) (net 12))
 (segment (start 103.95 59.0042) (end 103.95 55.5752) (width 0.3556) (layer F.Cu) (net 12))
 (segment (start 143.1165 56.5277) (end 143.129 56.515) (width 0.3556) (layer F.Cu) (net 2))
 (segment (start 136.258 56.5404) (end 143.104 56.5404) (width 0.3556) (layer F.Cu) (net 2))
 (segment (start 143.104 56.5404) (end 143.1165 56.5277) (width 0.3556) (layer F.Cu) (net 2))
 (segment (start 130.023 56.5531) (end 136.246 56.5531) (width 0.3556) (layer F.Cu) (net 2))
 (segment (start 136.246 56.5531) (end 136.258 56.5404) (width 0.3556) (layer F.Cu) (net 2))
 (segment (start 116.967 83.9337) (end 116.967 86.995) (width 0.3556) (layer B.Cu) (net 20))
 (segment (start 116.974 83.9271) (end 116.967 83.9337) (width 0.3556) (layer B.Cu) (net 20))
 (segment (start 120.639 93.0384) (end 120.6389 93.0384) (width 0.3556) (layer F.Cu) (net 20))
 (segment (start 120.6389 93.0384) (end 119.137 93.0384) (width 0.3556) (layer F.Cu) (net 20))
 (segment (start 119.137 93.0384) (end 116.967 90.8685) (width 0.3556) (layer F.Cu) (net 20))
 (segment (start 116.967 90.8685) (end 116.967 86.995) (width 0.3556) (layer F.Cu) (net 20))
 (segment (start 120.015 64.135) (end 120.015 60.0075) (width 0.3556) (layer B.Cu) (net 20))
 (segment (start 120.015 60.0075) (end 120.015 54.61) (width 0.25) (layer F.Cu) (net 20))
 (segment (start 120.015 54.61) (end 120.612 54.0131) (width 0.25) (layer F.Cu) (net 20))
 (segment (start 120.612 54.0131) (end 122.403 54.0131) (width 0.25) (layer F.Cu) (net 20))
 (segment (start 117.424 68.6308) (end 120.015 66.04) (width 0.3556) (layer F.Cu) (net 20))
 (segment (start 120.015 66.04) (end 120.015 64.135) (width 0.3556) (layer F.Cu) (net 20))
 (segment (start 116.967 83.9337) (end 116.967 69.088) (width 0.3556) (layer F.Cu) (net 20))
 (segment (start 116.967 69.088) (end 117.424 68.6308) (width 0.3556) (layer F.Cu) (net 20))
 (segment (start 117.03 69.0245) (end 117.424 68.6308) (width 0.3556) (layer F.Cu) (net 20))
 (via (at 116.967 86.995) (size 0.6) (layers F.Cu B.Cu) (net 20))
 (via (at 120.015 64.135) (size 0.6) (layers F.Cu B.Cu) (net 20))
 (via (at 120.015 60.0075) (size 0.6) (layers F.Cu B.Cu) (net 20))
 (via (at 116.967 83.9337) (size 0.6) (layers F.Cu B.Cu) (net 20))
 (segment (start 69.4436 61.2394) (end 69.4436 81.3816) (width 0.3556) (layer F.Cu) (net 4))
 (segment (start 59.2836 61.2394) (end 49.0855 61.2394) (width 0.3556) (layer F.Cu) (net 3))
 (segment (start 44.0055 81.3435) (end 44.0436 81.3816) (width 0.25) (layer F.Cu) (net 5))
 (segment (start 44.0055 61.2292) (end 44.0055 81.3435) (width 0.3556) (layer F.Cu) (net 5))
 (segment (start 44.0436 97.1296) (end 52.9209 97.1296) (width 0.3556) (layer F.Cu) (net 6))
 (segment (start 52.9209 97.1296) (end 60.7949 89.2556) (width 0.3556) (layer F.Cu) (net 6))
 (segment (start 60.7949 89.2556) (end 69.4436 89.2556) (width 0.3556) (layer F.Cu) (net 6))
 (segment (start 120.6389 85.4184) (end 124.919 85.4184) (width 0.3556) (layer F.Cu) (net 17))
 (segment (start 124.919 85.4184) (end 130.023 80.3148) (width 0.3556) (layer F.Cu) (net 17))
 (segment (start 130.023 80.3148) (end 130.023 63.881) (width 0.3556) (layer F.Cu) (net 17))
 (segment (start 114.605 85.3948) (end 114.628 85.4184) (width 0.3556) (layer F.Cu) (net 17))
 (segment (start 114.628 85.4184) (end 120.6389 85.4184) (width 0.3556) (layer F.Cu) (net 17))
 (segment (start 130.023 62.5094) (end 130.023 62.3443) (width 0.3556) (layer F.Cu) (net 17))
 (segment (start 130.023 63.881) (end 130.023 62.5094) (width 0.3556) (layer F.Cu) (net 17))
 (segment (start 130.023 62.3443) (end 130.023 62.5094) (width 0.3556) (layer F.Cu) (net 17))
 (segment (start 130.023 61.8871) (end 130.023 62.3443) (width 0.3556) (layer F.Cu) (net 17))
 (segment (start 130.023 61.8871) (end 130.023 59.0931) (width 0.3556) (layer F.Cu) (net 17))
 (segment (start 129.794 62.1157) (end 130.023 61.8871) (width 0.3556) (layer F.Cu) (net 17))
 (segment (start 130.023 62.3443) (end 129.794 62.1157) (width 0.3556) (layer F.Cu) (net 17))
 (segment (start 114.11 59.0042) (end 117.602 59.0042) (width 0.3556) (layer F.Cu) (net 17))
 (segment (start 117.602 59.0042) (end 117.602 60.7314) (width 0.3556) (layer F.Cu) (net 17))
 (segment (start 117.602 60.7314) (end 118.986 62.1157) (width 0.3556) (layer F.Cu) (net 17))
 (segment (start 118.986 62.1157) (end 129.794 62.1157) (width 0.3556) (layer F.Cu) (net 17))
 (segment (start 130.023 59.0931) (end 127.851 59.0931) (width 0.3556) (layer F.Cu) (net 17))
 (segment (start 127.851 59.0931) (end 127 58.2422) (width 0.3556) (layer F.Cu) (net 17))
 (segment (start 127 58.2422) (end 127 54.864) (width 0.3556) (layer F.Cu) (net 17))
 (segment (start 127 54.864) (end 127.851 54.0131) (width 0.3556) (layer F.Cu) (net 17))
 (segment (start 127.851 54.0131) (end 130.023 54.0131) (width 0.3556) (layer F.Cu) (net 17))
 (segment (start 130.023 54.0131) (end 130.023 51.4731) (width 0.3556) (layer F.Cu) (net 17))
 (segment (start 142.24 98.1075) (end 140.97 98.1075) (width 0.3556) (layer F.Cu) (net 18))
 (segment (start 140.97 98.1075) (end 138.786 100.292) (width 0.3556) (layer F.Cu) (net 18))
 (segment (start 138.786 100.292) (end 138.532 100.546) (width 0.3556) (layer F.Cu) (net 18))
 (segment (start 138.532 100.546) (end 114.922 100.546) (width 0.3556) (layer F.Cu) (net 18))
 (segment (start 114.922 100.546) (end 109.144 94.7674) (width 0.3556) (layer F.Cu) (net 18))
 (segment (start 109.144 94.7674) (end 109.144 77.7748) (width 0.3556) (layer F.Cu) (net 18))
 (segment (start 143.5099 98.1075) (end 142.24 98.1075) (width 0.3556) (layer F.Cu) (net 18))
 (segment (start 142.24 98.1075) (end 140.9699 98.1075) (width 0.25) (layer F.Cu) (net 18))
 (segment (start 143.51 98.1075) (end 143.5099 98.1075) (width 0.3556) (layer F.Cu) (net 18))
 (segment (start 109.144 75.2348) (end 114.605 75.2348) (width 0.3556) (layer F.Cu) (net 19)))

